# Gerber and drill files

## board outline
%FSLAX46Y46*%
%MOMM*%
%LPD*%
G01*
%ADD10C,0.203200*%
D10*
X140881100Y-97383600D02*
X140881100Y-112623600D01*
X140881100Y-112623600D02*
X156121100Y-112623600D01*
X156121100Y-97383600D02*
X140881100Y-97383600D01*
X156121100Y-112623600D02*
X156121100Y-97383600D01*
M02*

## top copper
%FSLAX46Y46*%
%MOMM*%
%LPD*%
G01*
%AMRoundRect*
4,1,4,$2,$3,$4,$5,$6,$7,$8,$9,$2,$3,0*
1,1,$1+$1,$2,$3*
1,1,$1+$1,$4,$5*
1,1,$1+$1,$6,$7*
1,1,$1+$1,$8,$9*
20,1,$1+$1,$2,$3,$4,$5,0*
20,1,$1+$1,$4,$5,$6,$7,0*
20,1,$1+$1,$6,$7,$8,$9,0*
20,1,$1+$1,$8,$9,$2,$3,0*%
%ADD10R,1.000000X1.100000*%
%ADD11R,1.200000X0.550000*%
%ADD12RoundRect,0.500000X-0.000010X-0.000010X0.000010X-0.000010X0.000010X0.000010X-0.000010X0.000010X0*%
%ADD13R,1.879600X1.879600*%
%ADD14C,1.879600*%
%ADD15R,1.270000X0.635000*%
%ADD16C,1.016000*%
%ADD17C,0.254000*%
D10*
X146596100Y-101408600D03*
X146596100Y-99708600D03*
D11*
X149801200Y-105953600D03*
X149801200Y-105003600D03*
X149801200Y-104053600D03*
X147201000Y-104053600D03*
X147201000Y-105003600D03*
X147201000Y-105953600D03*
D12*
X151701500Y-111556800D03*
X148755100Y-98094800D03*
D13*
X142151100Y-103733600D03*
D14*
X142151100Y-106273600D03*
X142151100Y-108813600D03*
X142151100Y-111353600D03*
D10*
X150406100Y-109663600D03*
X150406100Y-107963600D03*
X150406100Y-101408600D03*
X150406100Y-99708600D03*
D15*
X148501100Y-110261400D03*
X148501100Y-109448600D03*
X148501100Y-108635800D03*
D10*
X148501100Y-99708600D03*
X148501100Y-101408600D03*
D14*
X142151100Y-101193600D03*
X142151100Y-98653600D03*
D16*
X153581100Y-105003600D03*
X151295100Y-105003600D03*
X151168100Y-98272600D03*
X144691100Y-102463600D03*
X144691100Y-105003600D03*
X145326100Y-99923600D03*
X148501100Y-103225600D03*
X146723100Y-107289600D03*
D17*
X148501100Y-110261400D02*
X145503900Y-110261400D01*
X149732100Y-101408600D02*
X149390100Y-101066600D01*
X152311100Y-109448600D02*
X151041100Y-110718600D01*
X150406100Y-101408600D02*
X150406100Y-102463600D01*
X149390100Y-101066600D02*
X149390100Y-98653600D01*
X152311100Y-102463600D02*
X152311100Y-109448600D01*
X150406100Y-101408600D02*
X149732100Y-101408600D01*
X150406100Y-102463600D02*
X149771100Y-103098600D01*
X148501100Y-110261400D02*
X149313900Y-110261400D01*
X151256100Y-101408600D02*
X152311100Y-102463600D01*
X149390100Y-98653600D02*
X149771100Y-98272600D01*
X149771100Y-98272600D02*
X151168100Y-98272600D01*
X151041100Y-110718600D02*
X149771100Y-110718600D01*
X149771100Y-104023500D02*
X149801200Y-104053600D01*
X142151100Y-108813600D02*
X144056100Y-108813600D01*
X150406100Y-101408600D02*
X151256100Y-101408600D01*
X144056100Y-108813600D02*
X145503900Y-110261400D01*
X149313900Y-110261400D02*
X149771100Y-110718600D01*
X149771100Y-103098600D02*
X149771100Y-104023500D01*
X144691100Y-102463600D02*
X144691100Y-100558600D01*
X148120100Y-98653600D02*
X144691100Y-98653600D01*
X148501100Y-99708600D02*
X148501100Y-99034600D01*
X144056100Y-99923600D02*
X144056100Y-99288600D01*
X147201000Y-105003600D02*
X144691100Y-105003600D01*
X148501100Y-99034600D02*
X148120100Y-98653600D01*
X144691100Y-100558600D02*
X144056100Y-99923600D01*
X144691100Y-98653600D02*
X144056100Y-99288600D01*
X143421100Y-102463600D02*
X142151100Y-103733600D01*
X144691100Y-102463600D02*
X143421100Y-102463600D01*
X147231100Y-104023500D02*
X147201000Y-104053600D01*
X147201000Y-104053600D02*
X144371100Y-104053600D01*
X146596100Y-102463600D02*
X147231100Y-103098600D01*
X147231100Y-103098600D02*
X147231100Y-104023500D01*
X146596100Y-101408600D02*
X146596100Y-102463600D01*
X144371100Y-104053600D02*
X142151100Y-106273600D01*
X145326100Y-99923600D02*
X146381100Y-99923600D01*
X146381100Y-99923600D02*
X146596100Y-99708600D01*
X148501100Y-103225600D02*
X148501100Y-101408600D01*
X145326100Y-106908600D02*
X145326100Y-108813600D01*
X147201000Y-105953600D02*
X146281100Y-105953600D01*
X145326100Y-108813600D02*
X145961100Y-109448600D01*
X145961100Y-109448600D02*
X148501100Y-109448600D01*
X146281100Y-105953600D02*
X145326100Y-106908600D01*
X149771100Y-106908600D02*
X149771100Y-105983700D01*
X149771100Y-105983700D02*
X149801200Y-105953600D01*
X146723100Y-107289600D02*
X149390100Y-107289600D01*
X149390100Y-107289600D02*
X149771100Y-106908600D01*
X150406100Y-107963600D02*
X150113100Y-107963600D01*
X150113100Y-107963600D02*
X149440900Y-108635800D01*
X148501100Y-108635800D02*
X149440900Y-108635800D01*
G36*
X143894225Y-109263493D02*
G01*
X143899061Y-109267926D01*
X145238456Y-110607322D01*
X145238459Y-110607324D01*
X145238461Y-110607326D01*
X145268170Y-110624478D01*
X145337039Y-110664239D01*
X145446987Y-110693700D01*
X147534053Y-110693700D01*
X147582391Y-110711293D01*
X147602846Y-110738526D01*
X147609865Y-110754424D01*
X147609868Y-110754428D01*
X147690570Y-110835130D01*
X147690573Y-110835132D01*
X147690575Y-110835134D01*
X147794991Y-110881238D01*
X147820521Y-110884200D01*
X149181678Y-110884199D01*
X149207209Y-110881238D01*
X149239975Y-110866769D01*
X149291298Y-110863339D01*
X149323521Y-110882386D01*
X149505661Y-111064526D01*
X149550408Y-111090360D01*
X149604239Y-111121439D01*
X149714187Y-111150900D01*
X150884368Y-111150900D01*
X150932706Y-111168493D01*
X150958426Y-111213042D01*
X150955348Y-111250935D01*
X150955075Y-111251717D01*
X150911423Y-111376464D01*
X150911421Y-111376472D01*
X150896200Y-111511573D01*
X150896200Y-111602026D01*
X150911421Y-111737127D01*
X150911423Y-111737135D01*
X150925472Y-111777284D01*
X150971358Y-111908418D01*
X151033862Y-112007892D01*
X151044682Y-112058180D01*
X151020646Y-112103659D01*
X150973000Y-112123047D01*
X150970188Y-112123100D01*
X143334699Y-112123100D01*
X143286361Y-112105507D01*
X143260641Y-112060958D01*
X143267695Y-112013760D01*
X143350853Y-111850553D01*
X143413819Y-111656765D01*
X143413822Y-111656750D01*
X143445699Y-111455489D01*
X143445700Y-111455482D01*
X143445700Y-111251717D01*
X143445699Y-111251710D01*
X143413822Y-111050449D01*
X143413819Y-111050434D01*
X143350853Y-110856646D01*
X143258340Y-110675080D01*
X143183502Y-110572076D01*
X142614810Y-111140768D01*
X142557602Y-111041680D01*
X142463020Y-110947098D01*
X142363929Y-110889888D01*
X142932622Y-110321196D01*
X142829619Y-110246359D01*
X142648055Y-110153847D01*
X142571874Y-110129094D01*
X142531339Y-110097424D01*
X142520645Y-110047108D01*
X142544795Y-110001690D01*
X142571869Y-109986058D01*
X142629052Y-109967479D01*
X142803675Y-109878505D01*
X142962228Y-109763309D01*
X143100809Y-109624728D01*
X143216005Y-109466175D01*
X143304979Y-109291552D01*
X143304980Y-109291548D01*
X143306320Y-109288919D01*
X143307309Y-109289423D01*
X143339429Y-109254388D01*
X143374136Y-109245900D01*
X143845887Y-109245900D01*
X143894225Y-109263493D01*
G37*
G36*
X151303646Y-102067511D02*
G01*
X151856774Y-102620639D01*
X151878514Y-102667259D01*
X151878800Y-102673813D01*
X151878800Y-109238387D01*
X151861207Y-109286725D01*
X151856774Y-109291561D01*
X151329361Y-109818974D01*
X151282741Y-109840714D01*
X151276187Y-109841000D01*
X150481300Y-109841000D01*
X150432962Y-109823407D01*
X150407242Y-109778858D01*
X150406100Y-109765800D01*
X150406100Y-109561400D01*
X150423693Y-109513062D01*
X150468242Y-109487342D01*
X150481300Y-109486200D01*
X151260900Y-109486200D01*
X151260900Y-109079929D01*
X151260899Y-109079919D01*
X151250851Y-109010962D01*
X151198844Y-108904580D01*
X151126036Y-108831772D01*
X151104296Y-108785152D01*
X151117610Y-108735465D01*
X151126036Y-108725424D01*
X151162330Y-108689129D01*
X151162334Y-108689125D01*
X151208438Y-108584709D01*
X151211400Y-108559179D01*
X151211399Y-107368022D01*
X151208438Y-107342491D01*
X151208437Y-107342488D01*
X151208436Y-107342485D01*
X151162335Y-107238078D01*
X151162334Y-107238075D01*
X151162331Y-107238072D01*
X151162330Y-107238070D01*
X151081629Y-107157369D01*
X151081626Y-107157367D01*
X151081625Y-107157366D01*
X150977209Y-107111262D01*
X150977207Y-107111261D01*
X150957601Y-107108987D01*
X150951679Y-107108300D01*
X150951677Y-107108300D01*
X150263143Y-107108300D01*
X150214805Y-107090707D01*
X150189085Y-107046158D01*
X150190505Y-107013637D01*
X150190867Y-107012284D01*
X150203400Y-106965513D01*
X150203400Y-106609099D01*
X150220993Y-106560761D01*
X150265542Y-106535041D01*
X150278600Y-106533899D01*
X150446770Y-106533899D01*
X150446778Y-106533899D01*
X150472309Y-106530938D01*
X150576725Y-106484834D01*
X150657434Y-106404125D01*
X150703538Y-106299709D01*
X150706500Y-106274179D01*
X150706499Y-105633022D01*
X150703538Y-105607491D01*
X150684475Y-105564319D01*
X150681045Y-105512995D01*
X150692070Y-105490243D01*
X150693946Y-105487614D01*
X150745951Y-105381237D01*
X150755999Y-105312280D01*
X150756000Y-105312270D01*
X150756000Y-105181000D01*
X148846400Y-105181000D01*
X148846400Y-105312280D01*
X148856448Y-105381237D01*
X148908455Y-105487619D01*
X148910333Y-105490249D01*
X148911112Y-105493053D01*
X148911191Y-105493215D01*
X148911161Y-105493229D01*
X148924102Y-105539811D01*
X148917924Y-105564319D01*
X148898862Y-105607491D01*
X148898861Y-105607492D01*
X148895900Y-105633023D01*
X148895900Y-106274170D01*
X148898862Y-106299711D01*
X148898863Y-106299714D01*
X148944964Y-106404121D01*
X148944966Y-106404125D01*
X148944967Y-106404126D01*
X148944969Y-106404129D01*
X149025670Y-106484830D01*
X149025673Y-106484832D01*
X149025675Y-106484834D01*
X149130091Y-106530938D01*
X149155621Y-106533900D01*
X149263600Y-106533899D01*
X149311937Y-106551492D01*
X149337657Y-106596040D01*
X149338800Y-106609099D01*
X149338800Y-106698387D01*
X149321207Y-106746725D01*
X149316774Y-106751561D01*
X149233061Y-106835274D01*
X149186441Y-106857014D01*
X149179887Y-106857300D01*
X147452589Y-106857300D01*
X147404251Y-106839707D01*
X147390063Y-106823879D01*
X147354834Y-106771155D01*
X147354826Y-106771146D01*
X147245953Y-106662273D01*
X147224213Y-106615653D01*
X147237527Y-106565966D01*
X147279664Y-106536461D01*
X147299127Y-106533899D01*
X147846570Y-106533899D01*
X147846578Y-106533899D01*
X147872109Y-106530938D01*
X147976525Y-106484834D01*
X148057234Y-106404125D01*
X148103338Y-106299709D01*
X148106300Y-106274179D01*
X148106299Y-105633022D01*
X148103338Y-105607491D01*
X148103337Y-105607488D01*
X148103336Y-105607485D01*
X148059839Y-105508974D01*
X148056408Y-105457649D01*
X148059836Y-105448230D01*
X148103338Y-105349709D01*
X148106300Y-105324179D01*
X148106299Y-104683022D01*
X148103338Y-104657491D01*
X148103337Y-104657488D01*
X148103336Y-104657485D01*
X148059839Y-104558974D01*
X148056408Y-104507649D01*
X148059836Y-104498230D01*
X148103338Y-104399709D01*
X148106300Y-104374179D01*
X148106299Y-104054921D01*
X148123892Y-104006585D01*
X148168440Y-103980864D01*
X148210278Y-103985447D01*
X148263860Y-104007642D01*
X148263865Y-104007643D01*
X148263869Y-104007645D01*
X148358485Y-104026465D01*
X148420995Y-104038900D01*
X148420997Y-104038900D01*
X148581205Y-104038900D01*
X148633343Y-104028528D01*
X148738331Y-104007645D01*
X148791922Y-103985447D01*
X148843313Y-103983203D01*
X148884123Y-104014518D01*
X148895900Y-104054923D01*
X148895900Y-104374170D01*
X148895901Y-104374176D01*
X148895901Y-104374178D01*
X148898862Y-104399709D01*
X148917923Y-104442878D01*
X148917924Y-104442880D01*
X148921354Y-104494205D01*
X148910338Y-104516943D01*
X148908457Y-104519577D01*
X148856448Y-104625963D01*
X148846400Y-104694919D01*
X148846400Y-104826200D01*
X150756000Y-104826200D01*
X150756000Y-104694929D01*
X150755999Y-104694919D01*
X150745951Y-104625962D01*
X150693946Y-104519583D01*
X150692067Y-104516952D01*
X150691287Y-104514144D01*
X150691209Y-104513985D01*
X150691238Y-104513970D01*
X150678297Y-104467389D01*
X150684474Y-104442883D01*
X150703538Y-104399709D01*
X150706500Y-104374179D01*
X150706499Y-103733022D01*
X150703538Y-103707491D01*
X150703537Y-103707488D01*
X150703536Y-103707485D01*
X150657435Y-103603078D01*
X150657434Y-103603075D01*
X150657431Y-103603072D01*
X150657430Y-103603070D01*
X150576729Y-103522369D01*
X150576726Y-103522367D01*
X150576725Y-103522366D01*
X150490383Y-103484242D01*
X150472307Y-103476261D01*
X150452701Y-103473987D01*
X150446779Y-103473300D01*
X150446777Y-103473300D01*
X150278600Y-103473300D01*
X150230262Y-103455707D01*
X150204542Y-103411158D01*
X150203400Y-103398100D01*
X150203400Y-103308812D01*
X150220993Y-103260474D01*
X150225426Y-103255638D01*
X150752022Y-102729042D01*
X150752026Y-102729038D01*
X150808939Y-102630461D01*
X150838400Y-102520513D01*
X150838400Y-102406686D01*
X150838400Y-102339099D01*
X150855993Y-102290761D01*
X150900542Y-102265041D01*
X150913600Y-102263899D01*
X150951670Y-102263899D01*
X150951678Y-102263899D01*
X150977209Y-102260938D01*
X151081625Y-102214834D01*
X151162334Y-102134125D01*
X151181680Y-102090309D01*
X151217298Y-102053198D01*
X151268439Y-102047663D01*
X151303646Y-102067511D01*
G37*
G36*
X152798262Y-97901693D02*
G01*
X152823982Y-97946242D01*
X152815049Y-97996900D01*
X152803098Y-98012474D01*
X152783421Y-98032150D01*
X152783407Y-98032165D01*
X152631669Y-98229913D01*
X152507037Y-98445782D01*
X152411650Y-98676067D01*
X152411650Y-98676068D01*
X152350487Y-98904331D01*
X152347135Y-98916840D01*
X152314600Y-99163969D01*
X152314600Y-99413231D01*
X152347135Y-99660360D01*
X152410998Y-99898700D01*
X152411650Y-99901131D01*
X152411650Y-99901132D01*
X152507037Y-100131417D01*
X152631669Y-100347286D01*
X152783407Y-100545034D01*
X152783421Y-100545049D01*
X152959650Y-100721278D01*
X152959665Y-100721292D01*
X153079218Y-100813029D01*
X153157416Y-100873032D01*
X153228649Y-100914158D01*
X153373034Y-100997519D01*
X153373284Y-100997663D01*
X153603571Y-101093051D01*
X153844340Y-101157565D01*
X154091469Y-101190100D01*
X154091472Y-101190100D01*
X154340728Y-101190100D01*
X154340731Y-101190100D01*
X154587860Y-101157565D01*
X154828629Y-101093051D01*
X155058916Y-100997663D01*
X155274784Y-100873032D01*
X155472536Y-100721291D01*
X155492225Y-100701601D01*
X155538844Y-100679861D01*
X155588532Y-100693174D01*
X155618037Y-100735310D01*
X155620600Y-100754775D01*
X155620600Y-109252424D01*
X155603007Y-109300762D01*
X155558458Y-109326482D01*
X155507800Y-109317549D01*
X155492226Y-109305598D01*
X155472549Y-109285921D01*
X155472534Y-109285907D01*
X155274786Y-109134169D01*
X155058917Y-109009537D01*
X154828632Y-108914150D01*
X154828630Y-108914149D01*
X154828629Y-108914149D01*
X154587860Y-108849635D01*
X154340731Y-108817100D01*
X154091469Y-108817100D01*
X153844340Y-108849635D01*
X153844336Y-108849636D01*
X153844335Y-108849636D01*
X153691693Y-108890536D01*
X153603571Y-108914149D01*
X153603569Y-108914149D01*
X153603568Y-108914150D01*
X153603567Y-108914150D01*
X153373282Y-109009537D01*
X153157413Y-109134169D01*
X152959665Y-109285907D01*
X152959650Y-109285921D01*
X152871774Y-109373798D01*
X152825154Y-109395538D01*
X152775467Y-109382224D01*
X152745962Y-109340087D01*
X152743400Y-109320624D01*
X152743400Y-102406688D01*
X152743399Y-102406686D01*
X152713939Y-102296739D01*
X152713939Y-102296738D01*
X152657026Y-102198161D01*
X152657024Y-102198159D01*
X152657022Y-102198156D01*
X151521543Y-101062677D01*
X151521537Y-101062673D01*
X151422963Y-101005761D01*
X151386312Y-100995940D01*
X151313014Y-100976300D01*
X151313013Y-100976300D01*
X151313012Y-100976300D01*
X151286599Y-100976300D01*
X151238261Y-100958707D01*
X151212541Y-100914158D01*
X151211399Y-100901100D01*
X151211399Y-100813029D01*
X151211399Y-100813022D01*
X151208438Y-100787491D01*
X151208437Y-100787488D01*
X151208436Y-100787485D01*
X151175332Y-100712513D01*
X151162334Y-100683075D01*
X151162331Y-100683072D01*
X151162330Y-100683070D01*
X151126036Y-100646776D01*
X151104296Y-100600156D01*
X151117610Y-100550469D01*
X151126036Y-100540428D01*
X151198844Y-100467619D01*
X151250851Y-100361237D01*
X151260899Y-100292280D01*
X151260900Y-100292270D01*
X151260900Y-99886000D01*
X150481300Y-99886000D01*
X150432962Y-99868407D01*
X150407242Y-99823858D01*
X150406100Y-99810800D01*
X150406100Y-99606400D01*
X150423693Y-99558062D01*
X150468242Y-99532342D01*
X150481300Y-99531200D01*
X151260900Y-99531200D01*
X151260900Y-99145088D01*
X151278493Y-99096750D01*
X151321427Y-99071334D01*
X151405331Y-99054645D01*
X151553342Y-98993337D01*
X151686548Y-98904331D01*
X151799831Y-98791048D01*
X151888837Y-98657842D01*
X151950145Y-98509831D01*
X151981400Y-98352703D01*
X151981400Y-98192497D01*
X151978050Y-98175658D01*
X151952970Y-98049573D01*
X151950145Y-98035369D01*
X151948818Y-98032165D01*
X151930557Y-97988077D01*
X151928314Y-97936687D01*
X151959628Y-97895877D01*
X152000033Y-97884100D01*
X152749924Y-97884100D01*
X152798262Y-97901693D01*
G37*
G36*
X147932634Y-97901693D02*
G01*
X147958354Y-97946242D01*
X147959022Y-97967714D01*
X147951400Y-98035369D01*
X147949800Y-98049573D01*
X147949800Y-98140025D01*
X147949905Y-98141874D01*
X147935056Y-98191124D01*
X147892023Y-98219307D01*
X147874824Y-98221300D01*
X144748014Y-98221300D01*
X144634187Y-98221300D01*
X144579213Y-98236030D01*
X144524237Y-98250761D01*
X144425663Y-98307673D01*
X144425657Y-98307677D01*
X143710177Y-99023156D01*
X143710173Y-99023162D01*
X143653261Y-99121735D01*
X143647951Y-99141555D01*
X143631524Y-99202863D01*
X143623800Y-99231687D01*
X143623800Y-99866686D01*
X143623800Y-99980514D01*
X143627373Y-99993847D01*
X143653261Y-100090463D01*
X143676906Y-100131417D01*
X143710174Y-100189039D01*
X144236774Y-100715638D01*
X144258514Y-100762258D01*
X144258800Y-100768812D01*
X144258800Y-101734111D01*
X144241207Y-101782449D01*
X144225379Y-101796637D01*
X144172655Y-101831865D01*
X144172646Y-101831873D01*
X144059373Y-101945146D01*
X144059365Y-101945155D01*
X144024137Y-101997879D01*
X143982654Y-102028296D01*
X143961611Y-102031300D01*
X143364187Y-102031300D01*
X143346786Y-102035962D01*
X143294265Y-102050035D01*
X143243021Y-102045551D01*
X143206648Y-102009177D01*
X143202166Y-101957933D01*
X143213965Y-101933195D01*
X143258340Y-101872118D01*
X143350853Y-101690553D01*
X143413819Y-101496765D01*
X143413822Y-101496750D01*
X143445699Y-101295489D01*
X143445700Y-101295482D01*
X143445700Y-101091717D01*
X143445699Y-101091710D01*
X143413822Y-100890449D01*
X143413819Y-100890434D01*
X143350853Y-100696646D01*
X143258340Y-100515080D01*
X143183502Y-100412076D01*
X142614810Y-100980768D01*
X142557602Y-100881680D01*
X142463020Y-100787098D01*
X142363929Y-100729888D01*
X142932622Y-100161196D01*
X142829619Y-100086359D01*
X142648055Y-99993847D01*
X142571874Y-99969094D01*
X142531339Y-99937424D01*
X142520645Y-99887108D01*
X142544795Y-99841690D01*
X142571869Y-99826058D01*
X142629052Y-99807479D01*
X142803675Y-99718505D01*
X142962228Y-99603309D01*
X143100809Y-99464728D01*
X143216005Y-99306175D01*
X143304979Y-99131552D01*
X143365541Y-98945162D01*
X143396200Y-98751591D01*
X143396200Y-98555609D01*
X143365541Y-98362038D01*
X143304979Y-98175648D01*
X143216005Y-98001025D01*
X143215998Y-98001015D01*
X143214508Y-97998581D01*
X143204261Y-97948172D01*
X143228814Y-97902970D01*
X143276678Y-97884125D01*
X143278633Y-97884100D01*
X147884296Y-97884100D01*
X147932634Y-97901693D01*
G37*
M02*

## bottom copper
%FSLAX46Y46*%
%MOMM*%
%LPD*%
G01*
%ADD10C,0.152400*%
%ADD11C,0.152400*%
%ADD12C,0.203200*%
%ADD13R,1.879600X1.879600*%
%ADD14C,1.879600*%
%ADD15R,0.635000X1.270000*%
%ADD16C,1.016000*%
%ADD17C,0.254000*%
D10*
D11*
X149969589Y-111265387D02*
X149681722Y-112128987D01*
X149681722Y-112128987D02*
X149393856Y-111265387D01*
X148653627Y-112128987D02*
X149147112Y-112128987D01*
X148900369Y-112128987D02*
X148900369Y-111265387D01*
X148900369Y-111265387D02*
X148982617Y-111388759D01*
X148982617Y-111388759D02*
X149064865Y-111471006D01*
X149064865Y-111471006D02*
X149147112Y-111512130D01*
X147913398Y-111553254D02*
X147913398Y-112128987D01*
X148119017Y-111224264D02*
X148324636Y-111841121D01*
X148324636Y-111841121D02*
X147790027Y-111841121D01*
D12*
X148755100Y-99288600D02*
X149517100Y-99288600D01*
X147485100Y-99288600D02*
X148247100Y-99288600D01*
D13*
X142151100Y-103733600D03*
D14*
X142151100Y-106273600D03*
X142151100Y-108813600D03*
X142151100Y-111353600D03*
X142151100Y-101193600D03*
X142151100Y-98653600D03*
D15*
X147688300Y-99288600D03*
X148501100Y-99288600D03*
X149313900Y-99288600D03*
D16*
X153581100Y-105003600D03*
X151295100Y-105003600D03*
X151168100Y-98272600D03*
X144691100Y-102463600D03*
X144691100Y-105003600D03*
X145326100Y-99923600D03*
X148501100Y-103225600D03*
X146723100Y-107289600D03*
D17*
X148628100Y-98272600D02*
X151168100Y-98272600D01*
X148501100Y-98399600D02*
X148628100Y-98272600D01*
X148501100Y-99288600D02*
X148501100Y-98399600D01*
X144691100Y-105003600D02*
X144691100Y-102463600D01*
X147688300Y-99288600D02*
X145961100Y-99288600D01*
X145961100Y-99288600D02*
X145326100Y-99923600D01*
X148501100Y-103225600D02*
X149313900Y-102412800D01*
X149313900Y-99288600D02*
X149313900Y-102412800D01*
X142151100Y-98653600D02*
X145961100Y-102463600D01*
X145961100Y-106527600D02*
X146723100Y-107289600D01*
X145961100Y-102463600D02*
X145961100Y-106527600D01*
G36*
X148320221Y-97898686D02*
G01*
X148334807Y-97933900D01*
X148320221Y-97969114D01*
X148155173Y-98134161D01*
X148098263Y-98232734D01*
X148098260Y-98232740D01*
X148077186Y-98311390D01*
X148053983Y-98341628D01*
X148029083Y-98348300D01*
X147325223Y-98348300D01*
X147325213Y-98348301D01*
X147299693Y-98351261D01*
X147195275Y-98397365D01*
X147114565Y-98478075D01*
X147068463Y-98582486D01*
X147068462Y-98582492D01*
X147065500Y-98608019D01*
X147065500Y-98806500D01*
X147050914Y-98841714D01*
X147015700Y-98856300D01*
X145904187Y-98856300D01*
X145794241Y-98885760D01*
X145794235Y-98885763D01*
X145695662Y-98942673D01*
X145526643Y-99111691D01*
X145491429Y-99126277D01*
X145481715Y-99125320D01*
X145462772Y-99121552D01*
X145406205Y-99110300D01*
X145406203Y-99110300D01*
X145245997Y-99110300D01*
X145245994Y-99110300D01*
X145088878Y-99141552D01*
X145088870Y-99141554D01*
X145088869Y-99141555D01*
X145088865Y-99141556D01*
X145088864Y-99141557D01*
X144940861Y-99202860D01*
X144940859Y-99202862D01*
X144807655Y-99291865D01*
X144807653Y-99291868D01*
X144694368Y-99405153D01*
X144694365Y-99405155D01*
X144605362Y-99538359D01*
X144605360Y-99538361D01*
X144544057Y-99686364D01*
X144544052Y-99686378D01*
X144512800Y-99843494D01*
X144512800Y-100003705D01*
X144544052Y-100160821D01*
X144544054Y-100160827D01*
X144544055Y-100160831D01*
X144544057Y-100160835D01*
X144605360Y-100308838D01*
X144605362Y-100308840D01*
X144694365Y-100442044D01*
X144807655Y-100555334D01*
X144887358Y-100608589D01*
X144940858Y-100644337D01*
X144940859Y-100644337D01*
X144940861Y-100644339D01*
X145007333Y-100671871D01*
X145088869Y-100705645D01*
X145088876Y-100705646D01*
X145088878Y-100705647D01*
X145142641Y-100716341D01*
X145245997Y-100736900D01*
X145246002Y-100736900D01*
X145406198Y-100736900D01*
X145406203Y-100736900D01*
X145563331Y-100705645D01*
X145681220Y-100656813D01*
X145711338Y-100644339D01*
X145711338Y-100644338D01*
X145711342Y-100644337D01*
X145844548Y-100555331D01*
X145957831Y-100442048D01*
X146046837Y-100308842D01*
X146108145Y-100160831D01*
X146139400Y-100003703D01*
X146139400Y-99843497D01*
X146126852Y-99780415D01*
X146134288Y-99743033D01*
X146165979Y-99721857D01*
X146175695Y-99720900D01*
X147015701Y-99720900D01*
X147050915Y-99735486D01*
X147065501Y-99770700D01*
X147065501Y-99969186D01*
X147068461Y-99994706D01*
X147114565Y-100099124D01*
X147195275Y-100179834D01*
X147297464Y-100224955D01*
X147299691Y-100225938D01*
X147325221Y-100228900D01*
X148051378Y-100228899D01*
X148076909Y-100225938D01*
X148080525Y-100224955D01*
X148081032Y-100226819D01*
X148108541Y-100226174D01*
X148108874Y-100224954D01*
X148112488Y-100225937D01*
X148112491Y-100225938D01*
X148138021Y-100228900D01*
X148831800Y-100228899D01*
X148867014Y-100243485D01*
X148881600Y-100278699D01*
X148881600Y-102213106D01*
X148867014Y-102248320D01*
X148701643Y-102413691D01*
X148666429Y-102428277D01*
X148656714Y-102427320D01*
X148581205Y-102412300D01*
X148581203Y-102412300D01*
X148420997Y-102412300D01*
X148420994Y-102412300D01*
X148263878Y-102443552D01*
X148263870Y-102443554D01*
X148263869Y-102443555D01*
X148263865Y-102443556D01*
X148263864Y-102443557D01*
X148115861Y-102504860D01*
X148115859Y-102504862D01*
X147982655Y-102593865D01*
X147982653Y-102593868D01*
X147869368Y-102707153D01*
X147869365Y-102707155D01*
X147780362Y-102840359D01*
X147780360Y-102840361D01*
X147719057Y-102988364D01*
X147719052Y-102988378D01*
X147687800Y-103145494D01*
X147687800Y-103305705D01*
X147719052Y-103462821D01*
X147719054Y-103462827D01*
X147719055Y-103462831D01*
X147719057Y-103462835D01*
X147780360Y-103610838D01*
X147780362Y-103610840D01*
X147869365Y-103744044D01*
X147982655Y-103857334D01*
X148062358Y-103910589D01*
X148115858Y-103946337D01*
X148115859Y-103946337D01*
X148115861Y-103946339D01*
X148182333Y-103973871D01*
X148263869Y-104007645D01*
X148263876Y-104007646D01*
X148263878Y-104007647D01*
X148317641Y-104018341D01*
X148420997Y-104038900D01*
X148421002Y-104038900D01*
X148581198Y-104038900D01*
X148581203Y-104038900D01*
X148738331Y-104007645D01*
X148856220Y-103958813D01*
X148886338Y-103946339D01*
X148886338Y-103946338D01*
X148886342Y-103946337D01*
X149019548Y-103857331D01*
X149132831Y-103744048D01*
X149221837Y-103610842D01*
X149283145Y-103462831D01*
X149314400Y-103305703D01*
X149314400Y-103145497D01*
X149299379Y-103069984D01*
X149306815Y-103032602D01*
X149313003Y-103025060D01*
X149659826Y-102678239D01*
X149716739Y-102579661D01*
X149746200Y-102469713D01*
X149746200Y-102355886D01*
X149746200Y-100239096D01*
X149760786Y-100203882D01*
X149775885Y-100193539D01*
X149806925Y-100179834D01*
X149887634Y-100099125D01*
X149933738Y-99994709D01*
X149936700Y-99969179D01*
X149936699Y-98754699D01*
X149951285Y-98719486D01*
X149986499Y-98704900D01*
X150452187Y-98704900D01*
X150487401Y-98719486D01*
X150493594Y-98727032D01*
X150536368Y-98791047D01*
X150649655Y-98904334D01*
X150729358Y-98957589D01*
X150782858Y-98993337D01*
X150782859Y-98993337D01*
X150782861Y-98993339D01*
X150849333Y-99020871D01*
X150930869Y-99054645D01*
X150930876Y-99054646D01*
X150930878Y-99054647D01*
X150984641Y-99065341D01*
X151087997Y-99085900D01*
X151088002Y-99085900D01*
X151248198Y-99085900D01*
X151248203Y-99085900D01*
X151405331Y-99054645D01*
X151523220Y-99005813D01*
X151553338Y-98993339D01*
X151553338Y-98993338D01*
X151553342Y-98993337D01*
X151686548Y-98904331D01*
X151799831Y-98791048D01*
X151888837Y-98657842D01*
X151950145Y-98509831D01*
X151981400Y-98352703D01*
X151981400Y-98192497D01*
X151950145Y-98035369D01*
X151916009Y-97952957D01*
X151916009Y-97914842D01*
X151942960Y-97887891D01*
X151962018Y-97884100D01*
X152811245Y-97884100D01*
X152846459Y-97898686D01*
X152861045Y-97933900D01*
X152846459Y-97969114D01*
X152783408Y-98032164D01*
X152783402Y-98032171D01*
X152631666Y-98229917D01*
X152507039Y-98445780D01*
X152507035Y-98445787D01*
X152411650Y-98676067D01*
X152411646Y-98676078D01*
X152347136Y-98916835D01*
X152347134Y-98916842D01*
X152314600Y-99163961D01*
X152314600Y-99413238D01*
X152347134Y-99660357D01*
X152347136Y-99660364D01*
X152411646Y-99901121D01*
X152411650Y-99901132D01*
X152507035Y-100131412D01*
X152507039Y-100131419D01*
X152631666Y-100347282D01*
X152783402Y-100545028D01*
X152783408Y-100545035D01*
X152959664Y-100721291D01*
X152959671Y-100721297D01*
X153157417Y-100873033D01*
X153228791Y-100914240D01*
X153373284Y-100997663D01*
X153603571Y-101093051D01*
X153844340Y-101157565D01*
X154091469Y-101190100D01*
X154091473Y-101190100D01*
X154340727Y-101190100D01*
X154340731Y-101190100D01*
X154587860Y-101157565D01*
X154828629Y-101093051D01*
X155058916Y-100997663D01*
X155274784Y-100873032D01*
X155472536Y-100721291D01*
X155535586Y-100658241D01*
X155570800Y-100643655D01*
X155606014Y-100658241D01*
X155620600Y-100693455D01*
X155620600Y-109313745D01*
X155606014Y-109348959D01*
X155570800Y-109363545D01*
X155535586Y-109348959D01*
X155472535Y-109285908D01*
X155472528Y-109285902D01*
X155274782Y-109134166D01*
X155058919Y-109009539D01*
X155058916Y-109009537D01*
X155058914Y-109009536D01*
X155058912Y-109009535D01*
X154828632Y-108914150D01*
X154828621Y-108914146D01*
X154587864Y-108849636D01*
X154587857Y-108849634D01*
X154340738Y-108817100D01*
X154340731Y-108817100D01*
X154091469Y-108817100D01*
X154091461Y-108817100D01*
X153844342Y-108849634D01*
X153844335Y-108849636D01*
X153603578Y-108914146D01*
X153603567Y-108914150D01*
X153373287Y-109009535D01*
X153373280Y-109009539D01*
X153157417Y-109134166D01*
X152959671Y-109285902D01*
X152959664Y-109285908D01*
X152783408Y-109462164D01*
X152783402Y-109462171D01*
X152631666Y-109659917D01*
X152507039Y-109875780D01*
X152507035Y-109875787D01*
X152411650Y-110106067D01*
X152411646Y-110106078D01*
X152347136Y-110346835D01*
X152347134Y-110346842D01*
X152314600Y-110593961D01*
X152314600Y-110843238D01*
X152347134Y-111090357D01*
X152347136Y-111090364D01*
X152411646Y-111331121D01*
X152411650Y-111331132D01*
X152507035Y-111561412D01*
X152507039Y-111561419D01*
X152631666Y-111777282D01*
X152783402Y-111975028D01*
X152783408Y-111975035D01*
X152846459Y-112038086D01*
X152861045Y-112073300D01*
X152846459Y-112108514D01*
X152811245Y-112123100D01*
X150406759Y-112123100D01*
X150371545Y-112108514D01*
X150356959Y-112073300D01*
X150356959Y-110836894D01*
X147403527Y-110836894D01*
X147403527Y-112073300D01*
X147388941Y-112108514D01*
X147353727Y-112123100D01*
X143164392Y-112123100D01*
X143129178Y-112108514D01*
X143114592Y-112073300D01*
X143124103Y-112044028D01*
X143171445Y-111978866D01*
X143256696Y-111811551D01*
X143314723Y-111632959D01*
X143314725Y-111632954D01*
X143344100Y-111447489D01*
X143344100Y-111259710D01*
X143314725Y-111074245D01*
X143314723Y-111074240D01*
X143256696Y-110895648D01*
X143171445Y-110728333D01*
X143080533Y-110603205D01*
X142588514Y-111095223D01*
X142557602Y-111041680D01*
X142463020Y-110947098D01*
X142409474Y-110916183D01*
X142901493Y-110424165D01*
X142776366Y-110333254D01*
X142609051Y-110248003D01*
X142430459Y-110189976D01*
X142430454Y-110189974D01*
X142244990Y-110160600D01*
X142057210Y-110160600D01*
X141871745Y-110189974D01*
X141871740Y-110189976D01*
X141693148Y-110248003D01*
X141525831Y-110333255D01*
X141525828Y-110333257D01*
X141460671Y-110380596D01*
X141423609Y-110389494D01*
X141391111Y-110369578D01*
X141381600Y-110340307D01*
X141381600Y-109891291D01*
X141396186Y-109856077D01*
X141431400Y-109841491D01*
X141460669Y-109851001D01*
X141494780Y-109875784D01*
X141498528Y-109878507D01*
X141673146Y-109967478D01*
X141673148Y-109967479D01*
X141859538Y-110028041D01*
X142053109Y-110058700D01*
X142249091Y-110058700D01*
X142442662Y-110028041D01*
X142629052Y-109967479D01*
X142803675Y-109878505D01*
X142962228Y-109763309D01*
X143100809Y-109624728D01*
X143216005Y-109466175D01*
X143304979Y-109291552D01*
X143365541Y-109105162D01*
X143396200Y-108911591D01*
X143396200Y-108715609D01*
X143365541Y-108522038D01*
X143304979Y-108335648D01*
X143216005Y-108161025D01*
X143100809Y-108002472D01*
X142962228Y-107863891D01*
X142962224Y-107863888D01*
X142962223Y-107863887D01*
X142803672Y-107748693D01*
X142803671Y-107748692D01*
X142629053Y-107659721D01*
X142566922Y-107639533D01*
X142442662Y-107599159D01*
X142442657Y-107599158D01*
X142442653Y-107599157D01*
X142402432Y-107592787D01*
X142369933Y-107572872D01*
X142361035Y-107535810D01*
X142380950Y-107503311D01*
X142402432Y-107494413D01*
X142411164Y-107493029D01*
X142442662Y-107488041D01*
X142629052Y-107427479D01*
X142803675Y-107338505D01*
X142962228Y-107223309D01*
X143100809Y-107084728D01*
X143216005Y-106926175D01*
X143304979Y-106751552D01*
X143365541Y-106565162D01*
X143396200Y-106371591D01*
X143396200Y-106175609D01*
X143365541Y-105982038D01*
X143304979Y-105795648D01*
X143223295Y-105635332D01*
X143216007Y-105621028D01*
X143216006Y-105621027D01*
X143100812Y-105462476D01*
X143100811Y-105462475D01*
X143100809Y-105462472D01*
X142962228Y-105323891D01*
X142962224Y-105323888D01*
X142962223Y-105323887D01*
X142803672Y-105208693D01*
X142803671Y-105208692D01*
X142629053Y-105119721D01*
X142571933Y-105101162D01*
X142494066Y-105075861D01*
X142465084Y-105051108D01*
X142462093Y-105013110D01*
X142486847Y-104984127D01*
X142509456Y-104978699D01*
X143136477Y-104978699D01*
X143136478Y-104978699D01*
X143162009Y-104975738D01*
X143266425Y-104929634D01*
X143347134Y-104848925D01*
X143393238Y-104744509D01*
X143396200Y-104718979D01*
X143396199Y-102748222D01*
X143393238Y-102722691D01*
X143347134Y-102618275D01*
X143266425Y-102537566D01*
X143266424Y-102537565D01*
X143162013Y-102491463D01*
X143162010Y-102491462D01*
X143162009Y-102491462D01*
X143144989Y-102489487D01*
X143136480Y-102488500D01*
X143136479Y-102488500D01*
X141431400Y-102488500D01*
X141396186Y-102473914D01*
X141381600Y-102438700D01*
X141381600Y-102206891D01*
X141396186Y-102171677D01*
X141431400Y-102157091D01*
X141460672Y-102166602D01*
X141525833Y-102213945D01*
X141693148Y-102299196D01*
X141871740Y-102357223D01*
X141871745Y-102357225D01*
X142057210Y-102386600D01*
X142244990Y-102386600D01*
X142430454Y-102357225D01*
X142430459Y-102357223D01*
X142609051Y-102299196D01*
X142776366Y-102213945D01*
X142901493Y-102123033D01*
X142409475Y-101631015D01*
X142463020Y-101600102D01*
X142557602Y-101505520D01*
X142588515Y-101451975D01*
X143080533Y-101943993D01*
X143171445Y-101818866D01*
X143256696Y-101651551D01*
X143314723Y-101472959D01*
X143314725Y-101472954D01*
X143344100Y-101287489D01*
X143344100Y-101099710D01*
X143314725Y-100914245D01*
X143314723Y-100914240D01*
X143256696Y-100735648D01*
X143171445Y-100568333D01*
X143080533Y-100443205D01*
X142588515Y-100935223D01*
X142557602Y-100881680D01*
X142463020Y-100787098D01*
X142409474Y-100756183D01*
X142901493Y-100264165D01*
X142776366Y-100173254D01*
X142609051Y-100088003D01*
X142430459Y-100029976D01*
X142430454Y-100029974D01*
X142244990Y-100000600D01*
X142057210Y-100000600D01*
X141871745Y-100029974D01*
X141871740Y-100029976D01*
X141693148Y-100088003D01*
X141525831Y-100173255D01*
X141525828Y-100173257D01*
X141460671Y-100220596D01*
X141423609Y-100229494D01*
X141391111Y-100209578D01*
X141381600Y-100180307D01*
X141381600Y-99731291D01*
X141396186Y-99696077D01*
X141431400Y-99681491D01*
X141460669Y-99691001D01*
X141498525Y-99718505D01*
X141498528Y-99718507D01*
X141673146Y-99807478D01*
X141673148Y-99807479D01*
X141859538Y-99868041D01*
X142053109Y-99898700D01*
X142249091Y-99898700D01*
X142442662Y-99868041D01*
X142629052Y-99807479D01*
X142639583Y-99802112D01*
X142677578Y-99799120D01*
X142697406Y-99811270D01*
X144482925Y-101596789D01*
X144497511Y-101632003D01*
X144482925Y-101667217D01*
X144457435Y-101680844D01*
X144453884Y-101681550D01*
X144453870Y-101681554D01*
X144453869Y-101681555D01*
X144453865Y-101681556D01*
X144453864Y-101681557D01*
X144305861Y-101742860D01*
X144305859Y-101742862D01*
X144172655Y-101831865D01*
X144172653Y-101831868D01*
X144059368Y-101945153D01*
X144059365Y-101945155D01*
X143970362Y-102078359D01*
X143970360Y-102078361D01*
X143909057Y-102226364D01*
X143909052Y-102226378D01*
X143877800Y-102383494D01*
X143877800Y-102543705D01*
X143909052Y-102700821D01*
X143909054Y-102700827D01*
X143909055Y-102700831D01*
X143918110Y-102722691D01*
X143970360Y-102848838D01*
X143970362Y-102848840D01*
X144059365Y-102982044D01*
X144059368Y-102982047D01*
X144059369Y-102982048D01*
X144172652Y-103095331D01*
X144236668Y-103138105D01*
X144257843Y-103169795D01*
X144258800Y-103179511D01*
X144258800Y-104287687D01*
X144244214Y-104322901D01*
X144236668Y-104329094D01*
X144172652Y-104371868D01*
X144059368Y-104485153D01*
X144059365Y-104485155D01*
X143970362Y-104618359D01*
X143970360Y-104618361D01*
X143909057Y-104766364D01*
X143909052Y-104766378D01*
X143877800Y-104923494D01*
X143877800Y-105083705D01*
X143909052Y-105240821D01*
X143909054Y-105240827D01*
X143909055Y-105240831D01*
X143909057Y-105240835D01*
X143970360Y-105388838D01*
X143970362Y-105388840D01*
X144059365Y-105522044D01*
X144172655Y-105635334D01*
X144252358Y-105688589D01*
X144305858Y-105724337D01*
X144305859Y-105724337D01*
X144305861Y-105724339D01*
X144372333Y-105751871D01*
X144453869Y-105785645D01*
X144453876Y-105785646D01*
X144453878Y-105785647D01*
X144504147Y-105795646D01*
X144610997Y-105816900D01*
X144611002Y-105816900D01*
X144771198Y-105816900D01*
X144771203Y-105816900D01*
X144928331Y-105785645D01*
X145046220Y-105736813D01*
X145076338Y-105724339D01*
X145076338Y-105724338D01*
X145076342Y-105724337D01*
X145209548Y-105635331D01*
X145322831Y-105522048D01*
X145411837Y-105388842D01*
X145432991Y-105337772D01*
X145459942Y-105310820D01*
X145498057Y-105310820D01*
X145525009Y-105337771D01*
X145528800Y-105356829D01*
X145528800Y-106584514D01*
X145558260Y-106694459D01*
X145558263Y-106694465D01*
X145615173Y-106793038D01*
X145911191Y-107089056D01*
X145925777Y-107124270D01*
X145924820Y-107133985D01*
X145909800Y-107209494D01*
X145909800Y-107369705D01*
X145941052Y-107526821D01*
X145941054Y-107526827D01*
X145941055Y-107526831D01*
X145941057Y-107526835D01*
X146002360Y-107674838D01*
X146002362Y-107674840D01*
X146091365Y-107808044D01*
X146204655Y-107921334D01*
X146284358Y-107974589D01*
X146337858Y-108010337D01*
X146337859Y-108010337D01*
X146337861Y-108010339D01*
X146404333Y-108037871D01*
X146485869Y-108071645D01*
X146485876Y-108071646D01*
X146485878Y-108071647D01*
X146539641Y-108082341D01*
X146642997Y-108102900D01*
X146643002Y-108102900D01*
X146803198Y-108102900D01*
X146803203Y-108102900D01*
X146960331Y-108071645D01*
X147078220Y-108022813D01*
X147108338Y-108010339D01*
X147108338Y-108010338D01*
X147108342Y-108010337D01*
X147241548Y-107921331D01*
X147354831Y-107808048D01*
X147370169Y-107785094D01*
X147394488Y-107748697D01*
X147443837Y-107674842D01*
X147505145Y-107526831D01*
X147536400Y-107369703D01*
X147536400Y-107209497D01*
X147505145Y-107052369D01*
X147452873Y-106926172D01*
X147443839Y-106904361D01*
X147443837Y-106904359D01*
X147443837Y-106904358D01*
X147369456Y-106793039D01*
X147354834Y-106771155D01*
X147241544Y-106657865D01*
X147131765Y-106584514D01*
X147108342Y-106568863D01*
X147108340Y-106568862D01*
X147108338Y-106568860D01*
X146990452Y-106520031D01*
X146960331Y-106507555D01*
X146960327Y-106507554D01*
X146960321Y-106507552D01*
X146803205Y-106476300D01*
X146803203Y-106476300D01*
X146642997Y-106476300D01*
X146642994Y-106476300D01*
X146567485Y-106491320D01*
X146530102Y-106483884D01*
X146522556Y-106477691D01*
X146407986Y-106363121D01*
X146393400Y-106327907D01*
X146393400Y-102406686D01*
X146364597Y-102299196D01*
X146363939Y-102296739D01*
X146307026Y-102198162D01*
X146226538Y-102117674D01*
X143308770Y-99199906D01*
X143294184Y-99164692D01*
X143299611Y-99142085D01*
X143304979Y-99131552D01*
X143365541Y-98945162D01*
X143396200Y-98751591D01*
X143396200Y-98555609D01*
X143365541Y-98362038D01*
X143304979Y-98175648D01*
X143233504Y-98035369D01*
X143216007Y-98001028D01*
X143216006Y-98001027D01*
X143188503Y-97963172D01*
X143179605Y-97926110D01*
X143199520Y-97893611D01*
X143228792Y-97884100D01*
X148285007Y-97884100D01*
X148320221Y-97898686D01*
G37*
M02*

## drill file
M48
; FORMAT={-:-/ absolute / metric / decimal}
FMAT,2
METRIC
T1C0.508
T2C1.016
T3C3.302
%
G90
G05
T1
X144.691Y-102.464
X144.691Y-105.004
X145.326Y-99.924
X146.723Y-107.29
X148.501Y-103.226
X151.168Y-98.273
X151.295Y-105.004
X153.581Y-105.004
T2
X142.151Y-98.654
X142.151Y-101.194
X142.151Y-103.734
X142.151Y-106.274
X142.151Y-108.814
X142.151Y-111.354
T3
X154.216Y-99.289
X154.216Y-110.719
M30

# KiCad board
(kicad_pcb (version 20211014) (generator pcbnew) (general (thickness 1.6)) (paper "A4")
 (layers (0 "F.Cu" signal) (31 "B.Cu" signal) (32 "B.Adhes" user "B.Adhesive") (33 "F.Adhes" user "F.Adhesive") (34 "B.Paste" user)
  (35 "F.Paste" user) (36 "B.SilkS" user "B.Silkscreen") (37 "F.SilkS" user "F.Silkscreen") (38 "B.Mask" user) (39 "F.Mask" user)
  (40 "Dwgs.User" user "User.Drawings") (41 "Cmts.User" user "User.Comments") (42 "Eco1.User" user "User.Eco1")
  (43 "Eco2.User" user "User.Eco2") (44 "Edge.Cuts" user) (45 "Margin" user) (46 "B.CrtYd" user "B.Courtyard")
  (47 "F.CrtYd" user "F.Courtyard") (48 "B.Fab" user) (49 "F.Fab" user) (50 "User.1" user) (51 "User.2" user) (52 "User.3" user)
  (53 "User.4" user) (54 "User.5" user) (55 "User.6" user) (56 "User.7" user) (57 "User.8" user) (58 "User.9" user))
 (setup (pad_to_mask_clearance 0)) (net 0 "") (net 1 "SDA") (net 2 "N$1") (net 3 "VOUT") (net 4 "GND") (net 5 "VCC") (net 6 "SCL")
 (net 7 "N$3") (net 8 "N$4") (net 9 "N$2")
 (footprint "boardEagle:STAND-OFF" (layer "F.Cu") (at 154.2161 110.7186)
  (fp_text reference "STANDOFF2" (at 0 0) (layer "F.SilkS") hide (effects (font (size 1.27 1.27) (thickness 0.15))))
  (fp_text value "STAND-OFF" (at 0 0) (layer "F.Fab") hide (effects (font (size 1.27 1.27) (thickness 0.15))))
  (pad "" np_thru_hole circle (at 0 0) (size 3.302 3.302) (drill 3.302) (layers *.Cu *.Mask)))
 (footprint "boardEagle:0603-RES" (layer "F.Cu") (at 146.5961 100.5586 90)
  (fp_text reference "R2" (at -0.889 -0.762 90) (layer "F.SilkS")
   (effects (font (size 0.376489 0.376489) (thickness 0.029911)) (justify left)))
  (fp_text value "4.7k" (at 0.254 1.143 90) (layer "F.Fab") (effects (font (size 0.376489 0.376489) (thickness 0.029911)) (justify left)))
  (pad "1" smd rect (at -0.85 0 90) (size 1.1 1) (layers "F.Cu" "F.Paste" "F.Mask") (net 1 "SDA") (solder_mask_margin 0.1016))
  (pad "2" smd rect (at 0.85 0 90) (size 1.1 1) (layers "F.Cu" "F.Paste" "F.Mask") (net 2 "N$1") (solder_mask_margin 0.1016)))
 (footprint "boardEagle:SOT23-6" (layer "F.Cu") (at 148.5011 105.0036 -90)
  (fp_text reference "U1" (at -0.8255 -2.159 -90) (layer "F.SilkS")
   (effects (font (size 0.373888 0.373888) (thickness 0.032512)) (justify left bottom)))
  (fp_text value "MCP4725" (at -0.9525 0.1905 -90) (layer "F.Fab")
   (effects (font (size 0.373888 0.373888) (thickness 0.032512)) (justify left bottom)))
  (pad "1" smd rect (at 0.95 -1.3001 270) (size 0.55 1.2) (layers "F.Cu" "F.Paste" "F.Mask") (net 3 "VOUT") (solder_mask_margin 0.1016))
  (pad "2" smd rect (at 0 -1.3001 90) (size 0.55 1.2) (layers "F.Cu" "F.Paste" "F.Mask") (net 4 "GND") (solder_mask_margin 0.1016))
  (pad "3" smd rect (at -0.95 -1.3001 270) (size 0.55 1.2) (layers "F.Cu" "F.Paste" "F.Mask") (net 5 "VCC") (solder_mask_margin 0.1016))
  (pad "4" smd rect (at -0.95 1.3001 270) (size 0.55 1.2) (layers "F.Cu" "F.Paste" "F.Mask") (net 1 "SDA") (solder_mask_margin 0.1016))
  (pad "5" smd rect (at 0 1.3001 270) (size 0.55 1.2) (layers "F.Cu" "F.Paste" "F.Mask") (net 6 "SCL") (solder_mask_margin 0.1016))
  (pad "6" smd rect (at 0.95 1.3001 270) (size 0.55 1.2) (layers "F.Cu" "F.Paste" "F.Mask") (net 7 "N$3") (solder_mask_margin 0.1016)))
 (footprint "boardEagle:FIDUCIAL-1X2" (layer "F.Cu") (at 151.7015 111.5568)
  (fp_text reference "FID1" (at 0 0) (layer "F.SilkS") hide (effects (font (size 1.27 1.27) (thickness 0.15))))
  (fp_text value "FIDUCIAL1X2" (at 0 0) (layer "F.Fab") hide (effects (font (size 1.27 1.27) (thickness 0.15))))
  (pad "1" smd roundrect (at 0 0) (size 1 1) (layers "F.Cu" "F.Mask") (roundrect_rratio 0.5) (solder_mask_margin 0.1016)))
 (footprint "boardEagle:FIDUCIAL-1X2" (layer "F.Cu") (at 148.7551 98.0948)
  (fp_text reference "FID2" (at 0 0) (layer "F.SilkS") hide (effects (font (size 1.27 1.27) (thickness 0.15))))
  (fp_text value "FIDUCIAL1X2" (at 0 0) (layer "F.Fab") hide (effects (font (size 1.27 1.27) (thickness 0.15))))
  (pad "1" smd roundrect (at 0 0) (size 1 1) (layers "F.Cu" "F.Mask") (roundrect_rratio 0.5) (solder_mask_margin 0.1016)))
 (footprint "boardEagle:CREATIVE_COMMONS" (layer "F.Cu") (at 162.4711 134.2136)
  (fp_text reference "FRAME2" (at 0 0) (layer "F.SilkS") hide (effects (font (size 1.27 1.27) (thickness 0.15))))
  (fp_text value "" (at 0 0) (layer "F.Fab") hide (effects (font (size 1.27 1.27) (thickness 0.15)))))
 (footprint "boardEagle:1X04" (layer "F.Cu") (at 142.1511 103.7336 -90)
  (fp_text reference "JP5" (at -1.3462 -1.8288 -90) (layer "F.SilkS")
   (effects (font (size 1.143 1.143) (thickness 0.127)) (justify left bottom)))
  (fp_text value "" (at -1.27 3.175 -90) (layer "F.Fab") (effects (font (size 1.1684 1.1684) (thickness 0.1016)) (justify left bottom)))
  (pad "1" thru_hole rect (at 0 0) (size 1.8796 1.8796) (drill 1.016) (layers *.Cu *.Mask) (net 6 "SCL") (solder_mask_margin 0.1016))
  (pad "2" thru_hole circle (at 2.54 0) (size 1.8796 1.8796) (drill 1.016) (layers *.Cu *.Mask) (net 1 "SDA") (solder_mask_margin 0.1016))
  (pad "3" thru_hole circle (at 5.08 0) (size 1.8796 1.8796) (drill 1.016) (layers *.Cu *.Mask) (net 5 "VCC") (solder_mask_margin 0.1016))
  (pad "4" thru_hole circle (at 7.62 0) (size 1.8796 1.8796) (drill 1.016) (layers *.Cu *.Mask) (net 4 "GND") (solder_mask_margin 0.1016)))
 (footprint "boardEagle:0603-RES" (layer "F.Cu") (at 150.4061 108.8136 90)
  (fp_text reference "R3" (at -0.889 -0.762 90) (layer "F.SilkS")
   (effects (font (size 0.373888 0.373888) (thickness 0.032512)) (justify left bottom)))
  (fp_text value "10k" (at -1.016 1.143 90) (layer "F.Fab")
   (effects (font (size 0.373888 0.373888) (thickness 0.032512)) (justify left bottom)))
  (pad "1" smd rect (at -0.85 0 90) (size 1.1 1) (layers "F.Cu" "F.Paste" "F.Mask") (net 4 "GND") (solder_mask_margin 0.1016))
  (pad "2" smd rect (at 0.85 0 90) (size 1.1 1) (layers "F.Cu" "F.Paste" "F.Mask") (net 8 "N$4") (solder_mask_margin 0.1016)))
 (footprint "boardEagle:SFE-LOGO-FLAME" (layer "F.Cu") (at 151.2951 105.8926 -90)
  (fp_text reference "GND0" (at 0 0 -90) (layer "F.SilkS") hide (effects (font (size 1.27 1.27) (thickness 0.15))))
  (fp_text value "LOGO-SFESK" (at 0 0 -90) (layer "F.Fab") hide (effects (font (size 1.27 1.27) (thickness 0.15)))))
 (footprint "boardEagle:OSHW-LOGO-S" (layer "F.Cu") (at 152.3111 103.0986 -90)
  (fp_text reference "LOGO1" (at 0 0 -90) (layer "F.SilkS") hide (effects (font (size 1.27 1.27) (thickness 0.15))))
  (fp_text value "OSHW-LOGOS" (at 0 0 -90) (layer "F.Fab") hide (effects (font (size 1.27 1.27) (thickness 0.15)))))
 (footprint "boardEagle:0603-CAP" (layer "F.Cu") (at 150.4061 100.5586 90)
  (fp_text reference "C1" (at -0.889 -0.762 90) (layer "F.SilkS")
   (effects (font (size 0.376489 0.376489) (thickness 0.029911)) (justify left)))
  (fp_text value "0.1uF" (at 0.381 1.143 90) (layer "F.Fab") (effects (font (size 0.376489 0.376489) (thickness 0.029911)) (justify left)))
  (pad "1" smd rect (at -0.85 0 90) (size 1.1 1) (layers "F.Cu" "F.Paste" "F.Mask") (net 5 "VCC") (solder_mask_margin 0.1016))
  (pad "2" smd rect (at 0.85 0 90) (size 1.1 1) (layers "F.Cu" "F.Paste" "F.Mask") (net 4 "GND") (solder_mask_margin 0.1016)))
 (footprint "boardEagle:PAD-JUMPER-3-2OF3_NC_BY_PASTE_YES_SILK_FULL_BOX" (layer "F.Cu") (at 148.5011 109.4486 90)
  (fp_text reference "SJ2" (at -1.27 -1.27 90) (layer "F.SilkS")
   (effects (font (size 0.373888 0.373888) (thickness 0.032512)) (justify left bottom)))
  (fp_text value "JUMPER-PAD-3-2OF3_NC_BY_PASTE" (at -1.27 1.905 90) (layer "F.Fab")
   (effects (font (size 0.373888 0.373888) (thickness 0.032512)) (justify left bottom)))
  (pad "1" smd rect (at -0.8128 0 90) (size 0.635 1.27) (layers "F.Cu" "F.Mask") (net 5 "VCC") (solder_mask_margin 0.1016))
  (pad "2" smd rect (at 0 0 90) (size 0.635 1.27) (layers "F.Cu" "F.Mask") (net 7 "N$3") (solder_mask_margin 0.1016))
  (pad "3" smd rect (at 0.8128 0 90) (size 0.635 1.27) (layers "F.Cu" "F.Mask") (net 8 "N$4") (solder_mask_margin 0.1016)))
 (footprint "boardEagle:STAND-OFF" (layer "F.Cu") (at 154.2161 99.2886)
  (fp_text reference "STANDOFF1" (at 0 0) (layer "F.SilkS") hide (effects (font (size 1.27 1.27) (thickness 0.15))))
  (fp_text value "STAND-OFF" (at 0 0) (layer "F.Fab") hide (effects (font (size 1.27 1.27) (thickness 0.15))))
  (pad "" np_thru_hole circle (at 0 0) (size 3.302 3.302) (drill 3.302) (layers *.Cu *.Mask)))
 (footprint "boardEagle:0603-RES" (layer "F.Cu") (at 148.5011 100.5586 -90)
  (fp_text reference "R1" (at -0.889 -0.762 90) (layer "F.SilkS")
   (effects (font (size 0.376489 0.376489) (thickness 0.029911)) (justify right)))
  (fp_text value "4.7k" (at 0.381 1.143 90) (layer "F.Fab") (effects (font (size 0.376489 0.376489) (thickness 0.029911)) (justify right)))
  (pad "1" smd rect (at -0.85 0 270) (size 1.1 1) (layers "F.Cu" "F.Paste" "F.Mask") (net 6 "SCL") (solder_mask_margin 0.1016))
  (pad "2" smd rect (at 0.85 0 270) (size 1.1 1) (layers "F.Cu" "F.Paste" "F.Mask") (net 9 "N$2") (solder_mask_margin 0.1016)))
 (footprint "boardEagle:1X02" (layer "F.Cu") (at 142.1511 101.1936 90)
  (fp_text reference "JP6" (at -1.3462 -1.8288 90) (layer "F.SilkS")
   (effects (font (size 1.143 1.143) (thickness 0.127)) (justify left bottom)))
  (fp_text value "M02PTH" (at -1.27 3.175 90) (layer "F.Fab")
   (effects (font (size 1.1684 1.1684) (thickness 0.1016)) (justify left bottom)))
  (pad "1" thru_hole circle (at 0 0 180) (size 1.8796 1.8796) (drill 1.016) (layers *.Cu *.Mask) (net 4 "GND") (solder_mask_margin 0.1016))
  (pad "2" thru_hole circle (at 2.54 0 180) (size 1.8796 1.8796) (drill 1.016) (layers *.Cu *.Mask) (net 3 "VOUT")
   (solder_mask_margin 0.1016)))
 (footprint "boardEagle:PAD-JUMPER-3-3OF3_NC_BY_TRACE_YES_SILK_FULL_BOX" (layer "B.Cu") (at 148.5011 99.2886)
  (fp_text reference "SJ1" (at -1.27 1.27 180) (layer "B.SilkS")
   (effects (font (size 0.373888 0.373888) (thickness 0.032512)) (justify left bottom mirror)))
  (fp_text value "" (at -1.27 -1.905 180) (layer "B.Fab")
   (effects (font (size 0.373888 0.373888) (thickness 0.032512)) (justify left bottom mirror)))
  (fp_line (start 0.254 0) (end 1.016 0) (layer "B.Cu") (width 0.2032))
  (fp_line (start -1.016 0) (end -0.254 0) (layer "B.Cu") (width 0.2032))
  (pad "1" smd rect (at -0.8128 0) (size 0.635 1.27) (layers "B.Cu" "B.Mask") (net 2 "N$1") (solder_mask_margin 0.1016))
  (pad "2" smd rect (at 0 0) (size 0.635 1.27) (layers "B.Cu" "B.Mask") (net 5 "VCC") (solder_mask_margin 0.1016))
  (pad "3" smd rect (at 0.8128 0) (size 0.635 1.27) (layers "B.Cu" "B.Mask") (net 9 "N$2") (solder_mask_margin 0.1016)))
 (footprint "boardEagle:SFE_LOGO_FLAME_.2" (layer "B.Cu") (at 151.0411 109.4486 180)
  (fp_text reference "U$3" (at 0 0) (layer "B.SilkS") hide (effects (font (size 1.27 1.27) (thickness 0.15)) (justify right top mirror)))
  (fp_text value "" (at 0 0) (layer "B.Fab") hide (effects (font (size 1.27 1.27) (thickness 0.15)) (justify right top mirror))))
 (gr_line (start 140.8811 97.3836) (end 140.8811 112.6236) (layer "Edge.Cuts") (width 0.2032))
 (gr_line (start 140.8811 112.6236) (end 156.1211 112.6236) (layer "Edge.Cuts") (width 0.2032))
 (gr_line (start 156.1211 97.3836) (end 140.8811 97.3836) (layer "Edge.Cuts") (width 0.2032))
 (gr_line (start 156.1211 112.6236) (end 156.1211 97.3836) (layer "Edge.Cuts") (width 0.2032))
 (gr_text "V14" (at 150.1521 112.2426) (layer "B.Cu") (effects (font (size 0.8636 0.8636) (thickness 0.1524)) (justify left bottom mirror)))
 (via (at 153.5811 105.0036) (size 1.016) (drill 0.508) (layers "F.Cu" "B.Cu") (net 4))
 (via (at 151.2951 105.0036) (size 1.016) (drill 0.508) (layers "F.Cu" "B.Cu") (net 4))
 (segment (start 148.5011 110.2614) (end 145.5039 110.2614) (width 0.254) (layer "F.Cu") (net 5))
 (segment (start 149.7321 101.4086) (end 149.3901 101.0666) (width 0.254) (layer "F.Cu") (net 5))
 (segment (start 152.3111 109.4486) (end 151.0411 110.7186) (width 0.254) (layer "F.Cu") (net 5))
 (segment (start 150.4061 101.4086) (end 150.4061 102.4636) (width 0.254) (layer "F.Cu") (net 5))
 (segment (start 149.3901 101.0666) (end 149.3901 98.6536) (width 0.254) (layer "F.Cu") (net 5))
 (segment (start 152.3111 102.4636) (end 152.3111 109.4486) (width 0.254) (layer "F.Cu") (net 5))
 (segment (start 150.4061 101.4086) (end 149.7321 101.4086) (width 0.254) (layer "F.Cu") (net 5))
 (segment (start 150.4061 102.4636) (end 149.7711 103.0986) (width 0.254) (layer "F.Cu") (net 5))
 (segment (start 148.5011 110.2614) (end 149.3139 110.2614) (width 0.254) (layer "F.Cu") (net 5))
 (segment (start 151.2561 101.4086) (end 152.3111 102.4636) (width 0.254) (layer "F.Cu") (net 5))
 (segment (start 149.3901 98.6536) (end 149.7711 98.2726) (width 0.254) (layer "F.Cu") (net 5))
 (segment (start 149.7711 98.2726) (end 151.1681 98.2726) (width 0.254) (layer "F.Cu") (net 5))
 (segment (start 151.0411 110.7186) (end 149.7711 110.7186) (width 0.254) (layer "F.Cu") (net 5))
 (segment (start 149.7711 104.0235) (end 149.8012 104.0536) (width 0.254) (layer "F.Cu") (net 5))
 (segment (start 142.1511 108.8136) (end 144.0561 108.8136) (width 0.254) (layer "F.Cu") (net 5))
 (segment (start 150.4061 101.4086) (end 151.2561 101.4086) (width 0.254) (layer "F.Cu") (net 5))
 (segment (start 144.0561 108.8136) (end 145.5039 110.2614) (width 0.254) (layer "F.Cu") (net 5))
 (segment (start 149.3139 110.2614) (end 149.7711 110.7186) (width 0.254) (layer "F.Cu") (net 5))
 (segment (start 149.7711 103.0986) (end 149.7711 104.0235) (width 0.254) (layer "F.Cu") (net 5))
 (via (at 151.1681 98.2726) (size 1.016) (drill 0.508) (layers "F.Cu" "B.Cu") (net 5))
 (segment (start 148.6281 98.2726) (end 151.1681 98.2726) (width 0.254) (layer "B.Cu") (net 5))
 (segment (start 148.5011 98.3996) (end 148.6281 98.2726) (width 0.254) (layer "B.Cu") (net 5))
 (segment (start 148.5011 99.2886) (end 148.5011 98.3996) (width 0.254) (layer "B.Cu") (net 5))
 (segment (start 144.6911 102.4636) (end 144.6911 100.5586) (width 0.254) (layer "F.Cu") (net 6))
 (segment (start 148.1201 98.6536) (end 144.6911 98.6536) (width 0.254) (layer "F.Cu") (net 6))
 (segment (start 148.5011 99.7086) (end 148.5011 99.0346) (width 0.254) (layer "F.Cu") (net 6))
 (segment (start 144.0561 99.9236) (end 144.0561 99.2886) (width 0.254) (layer "F.Cu") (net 6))
 (segment (start 147.201 105.0036) (end 144.6911 105.0036) (width 0.254) (layer "F.Cu") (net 6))
 (segment (start 148.5011 99.0346) (end 148.1201 98.6536) (width 0.254) (layer "F.Cu") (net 6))
 (segment (start 144.6911 100.5586) (end 144.0561 99.9236) (width 0.254) (layer "F.Cu") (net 6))
 (segment (start 144.6911 98.6536) (end 144.0561 99.2886) (width 0.254) (layer "F.Cu") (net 6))
 (segment (start 143.4211 102.4636) (end 142.1511 103.7336) (width 0.254) (layer "F.Cu") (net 6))
 (segment (start 144.6911 102.4636) (end 143.4211 102.4636) (width 0.254) (layer "F.Cu") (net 6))
 (via (at 144.6911 102.4636) (size 1.016) (drill 0.508) (layers "F.Cu" "B.Cu") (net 6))
 (via (at 144.6911 105.0036) (size 1.016) (drill 0.508) (layers "F.Cu" "B.Cu") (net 6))
 (segment (start 144.6911 105.0036) (end 144.6911 102.4636) (width 0.254) (layer "B.Cu") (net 6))
 (segment (start 147.2311 104.0235) (end 147.201 104.0536) (width 0.254) (layer "F.Cu") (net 1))
 (segment (start 147.201 104.0536) (end 144.3711 104.0536) (width 0.254) (layer "F.Cu") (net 1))
 (segment (start 146.5961 102.4636) (end 147.2311 103.0986) (width 0.254) (layer "F.Cu") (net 1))
 (segment (start 147.2311 103.0986) (end 147.2311 104.0235) (width 0.254) (layer "F.Cu") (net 1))
 (segment (start 146.5961 101.4086) (end 146.5961 102.4636) (width 0.254) (layer "F.Cu") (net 1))
 (segment (start 144.3711 104.0536) (end 142.1511 106.2736) (width 0.254) (layer "F.Cu") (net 1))
 (segment (start 145.3261 99.9236) (end 146.3811 99.9236) (width 0.254) (layer "F.Cu") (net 2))
 (segment (start 146.3811 99.9236) (end 146.5961 99.7086) (width 0.254) (layer "F.Cu") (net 2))
 (via (at 145.3261 99.9236) (size 1.016) (drill 0.508) (layers "F.Cu" "B.Cu") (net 2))
 (segment (start 147.6883 99.2886) (end 145.9611 99.2886) (width 0.254) (layer "B.Cu") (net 2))
 (segment (start 145.9611 99.2886) (end 145.3261 99.9236) (width 0.254) (layer "B.Cu") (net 2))
 (segment (start 148.5011 103.2256) (end 148.5011 101.4086) (width 0.254) (layer "F.Cu") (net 9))
 (via (at 148.5011 103.2256) (size 1.016) (drill 0.508) (layers "F.Cu" "B.Cu") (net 9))
 (segment (start 148.5011 103.2256) (end 149.3139 102.4128) (width 0.254) (layer "B.Cu") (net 9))
 (segment (start 149.3139 99.2886) (end 149.3139 102.4128) (width 0.254) (layer "B.Cu") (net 9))
 (segment (start 145.3261 106.9086) (end 145.3261 108.8136) (width 0.254) (layer "F.Cu") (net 7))
 (segment (start 147.201 105.9536) (end 146.2811 105.9536) (width 0.254) (layer "F.Cu") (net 7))
 (segment (start 145.3261 108.8136) (end 145.9611 109.4486) (width 0.254) (layer "F.Cu") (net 7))
 (segment (start 145.9611 109.4486) (end 148.5011 109.4486) (width 0.254) (layer "F.Cu") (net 7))
 (segment (start 146.2811 105.9536) (end 145.3261 106.9086) (width 0.254) (layer "F.Cu") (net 7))
 (segment (start 149.7711 106.9086) (end 149.7711 105.9837) (width 0.254) (layer "F.Cu") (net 3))
 (segment (start 149.7711 105.9837) (end 149.8012 105.9536) (width 0.254) (layer "F.Cu") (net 3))
 (segment (start 146.7231 107.2896) (end 149.3901 107.2896) (width 0.254) (layer "F.Cu") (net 3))
 (segment (start 149.3901 107.2896) (end 149.7711 106.9086) (width 0.254) (layer "F.Cu") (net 3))
 (via (at 146.7231 107.2896) (size 1.016) (drill 0.508) (layers "F.Cu" "B.Cu") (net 3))
 (segment (start 142.1511 98.6536) (end 145.9611 102.4636) (width 0.254) (layer "B.Cu") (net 3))
 (segment (start 145.9611 106.5276) (end 146.7231 107.2896) (width 0.254) (layer "B.Cu") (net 3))
 (segment (start 145.9611 102.4636) (end 145.9611 106.5276) (width 0.254) (layer "B.Cu") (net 3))
 (segment (start 150.4061 107.9636) (end 150.1131 107.9636) (width 0.254) (layer "F.Cu") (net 8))
 (segment (start 150.1131 107.9636) (end 149.4409 108.6358) (width 0.254) (layer "F.Cu") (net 8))
 (segment (start 148.5011 108.6358) (end 149.4409 108.6358) (width 0.254) (layer "F.Cu") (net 8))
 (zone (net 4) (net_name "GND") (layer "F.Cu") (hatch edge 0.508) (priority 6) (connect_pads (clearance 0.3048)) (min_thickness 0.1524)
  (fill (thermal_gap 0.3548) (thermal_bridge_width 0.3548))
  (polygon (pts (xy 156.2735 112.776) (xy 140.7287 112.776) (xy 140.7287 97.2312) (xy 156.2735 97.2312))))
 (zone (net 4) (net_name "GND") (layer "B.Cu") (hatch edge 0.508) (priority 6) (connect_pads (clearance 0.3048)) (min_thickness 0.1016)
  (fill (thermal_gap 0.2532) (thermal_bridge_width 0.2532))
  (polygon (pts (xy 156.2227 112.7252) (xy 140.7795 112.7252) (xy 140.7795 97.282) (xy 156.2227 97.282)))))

